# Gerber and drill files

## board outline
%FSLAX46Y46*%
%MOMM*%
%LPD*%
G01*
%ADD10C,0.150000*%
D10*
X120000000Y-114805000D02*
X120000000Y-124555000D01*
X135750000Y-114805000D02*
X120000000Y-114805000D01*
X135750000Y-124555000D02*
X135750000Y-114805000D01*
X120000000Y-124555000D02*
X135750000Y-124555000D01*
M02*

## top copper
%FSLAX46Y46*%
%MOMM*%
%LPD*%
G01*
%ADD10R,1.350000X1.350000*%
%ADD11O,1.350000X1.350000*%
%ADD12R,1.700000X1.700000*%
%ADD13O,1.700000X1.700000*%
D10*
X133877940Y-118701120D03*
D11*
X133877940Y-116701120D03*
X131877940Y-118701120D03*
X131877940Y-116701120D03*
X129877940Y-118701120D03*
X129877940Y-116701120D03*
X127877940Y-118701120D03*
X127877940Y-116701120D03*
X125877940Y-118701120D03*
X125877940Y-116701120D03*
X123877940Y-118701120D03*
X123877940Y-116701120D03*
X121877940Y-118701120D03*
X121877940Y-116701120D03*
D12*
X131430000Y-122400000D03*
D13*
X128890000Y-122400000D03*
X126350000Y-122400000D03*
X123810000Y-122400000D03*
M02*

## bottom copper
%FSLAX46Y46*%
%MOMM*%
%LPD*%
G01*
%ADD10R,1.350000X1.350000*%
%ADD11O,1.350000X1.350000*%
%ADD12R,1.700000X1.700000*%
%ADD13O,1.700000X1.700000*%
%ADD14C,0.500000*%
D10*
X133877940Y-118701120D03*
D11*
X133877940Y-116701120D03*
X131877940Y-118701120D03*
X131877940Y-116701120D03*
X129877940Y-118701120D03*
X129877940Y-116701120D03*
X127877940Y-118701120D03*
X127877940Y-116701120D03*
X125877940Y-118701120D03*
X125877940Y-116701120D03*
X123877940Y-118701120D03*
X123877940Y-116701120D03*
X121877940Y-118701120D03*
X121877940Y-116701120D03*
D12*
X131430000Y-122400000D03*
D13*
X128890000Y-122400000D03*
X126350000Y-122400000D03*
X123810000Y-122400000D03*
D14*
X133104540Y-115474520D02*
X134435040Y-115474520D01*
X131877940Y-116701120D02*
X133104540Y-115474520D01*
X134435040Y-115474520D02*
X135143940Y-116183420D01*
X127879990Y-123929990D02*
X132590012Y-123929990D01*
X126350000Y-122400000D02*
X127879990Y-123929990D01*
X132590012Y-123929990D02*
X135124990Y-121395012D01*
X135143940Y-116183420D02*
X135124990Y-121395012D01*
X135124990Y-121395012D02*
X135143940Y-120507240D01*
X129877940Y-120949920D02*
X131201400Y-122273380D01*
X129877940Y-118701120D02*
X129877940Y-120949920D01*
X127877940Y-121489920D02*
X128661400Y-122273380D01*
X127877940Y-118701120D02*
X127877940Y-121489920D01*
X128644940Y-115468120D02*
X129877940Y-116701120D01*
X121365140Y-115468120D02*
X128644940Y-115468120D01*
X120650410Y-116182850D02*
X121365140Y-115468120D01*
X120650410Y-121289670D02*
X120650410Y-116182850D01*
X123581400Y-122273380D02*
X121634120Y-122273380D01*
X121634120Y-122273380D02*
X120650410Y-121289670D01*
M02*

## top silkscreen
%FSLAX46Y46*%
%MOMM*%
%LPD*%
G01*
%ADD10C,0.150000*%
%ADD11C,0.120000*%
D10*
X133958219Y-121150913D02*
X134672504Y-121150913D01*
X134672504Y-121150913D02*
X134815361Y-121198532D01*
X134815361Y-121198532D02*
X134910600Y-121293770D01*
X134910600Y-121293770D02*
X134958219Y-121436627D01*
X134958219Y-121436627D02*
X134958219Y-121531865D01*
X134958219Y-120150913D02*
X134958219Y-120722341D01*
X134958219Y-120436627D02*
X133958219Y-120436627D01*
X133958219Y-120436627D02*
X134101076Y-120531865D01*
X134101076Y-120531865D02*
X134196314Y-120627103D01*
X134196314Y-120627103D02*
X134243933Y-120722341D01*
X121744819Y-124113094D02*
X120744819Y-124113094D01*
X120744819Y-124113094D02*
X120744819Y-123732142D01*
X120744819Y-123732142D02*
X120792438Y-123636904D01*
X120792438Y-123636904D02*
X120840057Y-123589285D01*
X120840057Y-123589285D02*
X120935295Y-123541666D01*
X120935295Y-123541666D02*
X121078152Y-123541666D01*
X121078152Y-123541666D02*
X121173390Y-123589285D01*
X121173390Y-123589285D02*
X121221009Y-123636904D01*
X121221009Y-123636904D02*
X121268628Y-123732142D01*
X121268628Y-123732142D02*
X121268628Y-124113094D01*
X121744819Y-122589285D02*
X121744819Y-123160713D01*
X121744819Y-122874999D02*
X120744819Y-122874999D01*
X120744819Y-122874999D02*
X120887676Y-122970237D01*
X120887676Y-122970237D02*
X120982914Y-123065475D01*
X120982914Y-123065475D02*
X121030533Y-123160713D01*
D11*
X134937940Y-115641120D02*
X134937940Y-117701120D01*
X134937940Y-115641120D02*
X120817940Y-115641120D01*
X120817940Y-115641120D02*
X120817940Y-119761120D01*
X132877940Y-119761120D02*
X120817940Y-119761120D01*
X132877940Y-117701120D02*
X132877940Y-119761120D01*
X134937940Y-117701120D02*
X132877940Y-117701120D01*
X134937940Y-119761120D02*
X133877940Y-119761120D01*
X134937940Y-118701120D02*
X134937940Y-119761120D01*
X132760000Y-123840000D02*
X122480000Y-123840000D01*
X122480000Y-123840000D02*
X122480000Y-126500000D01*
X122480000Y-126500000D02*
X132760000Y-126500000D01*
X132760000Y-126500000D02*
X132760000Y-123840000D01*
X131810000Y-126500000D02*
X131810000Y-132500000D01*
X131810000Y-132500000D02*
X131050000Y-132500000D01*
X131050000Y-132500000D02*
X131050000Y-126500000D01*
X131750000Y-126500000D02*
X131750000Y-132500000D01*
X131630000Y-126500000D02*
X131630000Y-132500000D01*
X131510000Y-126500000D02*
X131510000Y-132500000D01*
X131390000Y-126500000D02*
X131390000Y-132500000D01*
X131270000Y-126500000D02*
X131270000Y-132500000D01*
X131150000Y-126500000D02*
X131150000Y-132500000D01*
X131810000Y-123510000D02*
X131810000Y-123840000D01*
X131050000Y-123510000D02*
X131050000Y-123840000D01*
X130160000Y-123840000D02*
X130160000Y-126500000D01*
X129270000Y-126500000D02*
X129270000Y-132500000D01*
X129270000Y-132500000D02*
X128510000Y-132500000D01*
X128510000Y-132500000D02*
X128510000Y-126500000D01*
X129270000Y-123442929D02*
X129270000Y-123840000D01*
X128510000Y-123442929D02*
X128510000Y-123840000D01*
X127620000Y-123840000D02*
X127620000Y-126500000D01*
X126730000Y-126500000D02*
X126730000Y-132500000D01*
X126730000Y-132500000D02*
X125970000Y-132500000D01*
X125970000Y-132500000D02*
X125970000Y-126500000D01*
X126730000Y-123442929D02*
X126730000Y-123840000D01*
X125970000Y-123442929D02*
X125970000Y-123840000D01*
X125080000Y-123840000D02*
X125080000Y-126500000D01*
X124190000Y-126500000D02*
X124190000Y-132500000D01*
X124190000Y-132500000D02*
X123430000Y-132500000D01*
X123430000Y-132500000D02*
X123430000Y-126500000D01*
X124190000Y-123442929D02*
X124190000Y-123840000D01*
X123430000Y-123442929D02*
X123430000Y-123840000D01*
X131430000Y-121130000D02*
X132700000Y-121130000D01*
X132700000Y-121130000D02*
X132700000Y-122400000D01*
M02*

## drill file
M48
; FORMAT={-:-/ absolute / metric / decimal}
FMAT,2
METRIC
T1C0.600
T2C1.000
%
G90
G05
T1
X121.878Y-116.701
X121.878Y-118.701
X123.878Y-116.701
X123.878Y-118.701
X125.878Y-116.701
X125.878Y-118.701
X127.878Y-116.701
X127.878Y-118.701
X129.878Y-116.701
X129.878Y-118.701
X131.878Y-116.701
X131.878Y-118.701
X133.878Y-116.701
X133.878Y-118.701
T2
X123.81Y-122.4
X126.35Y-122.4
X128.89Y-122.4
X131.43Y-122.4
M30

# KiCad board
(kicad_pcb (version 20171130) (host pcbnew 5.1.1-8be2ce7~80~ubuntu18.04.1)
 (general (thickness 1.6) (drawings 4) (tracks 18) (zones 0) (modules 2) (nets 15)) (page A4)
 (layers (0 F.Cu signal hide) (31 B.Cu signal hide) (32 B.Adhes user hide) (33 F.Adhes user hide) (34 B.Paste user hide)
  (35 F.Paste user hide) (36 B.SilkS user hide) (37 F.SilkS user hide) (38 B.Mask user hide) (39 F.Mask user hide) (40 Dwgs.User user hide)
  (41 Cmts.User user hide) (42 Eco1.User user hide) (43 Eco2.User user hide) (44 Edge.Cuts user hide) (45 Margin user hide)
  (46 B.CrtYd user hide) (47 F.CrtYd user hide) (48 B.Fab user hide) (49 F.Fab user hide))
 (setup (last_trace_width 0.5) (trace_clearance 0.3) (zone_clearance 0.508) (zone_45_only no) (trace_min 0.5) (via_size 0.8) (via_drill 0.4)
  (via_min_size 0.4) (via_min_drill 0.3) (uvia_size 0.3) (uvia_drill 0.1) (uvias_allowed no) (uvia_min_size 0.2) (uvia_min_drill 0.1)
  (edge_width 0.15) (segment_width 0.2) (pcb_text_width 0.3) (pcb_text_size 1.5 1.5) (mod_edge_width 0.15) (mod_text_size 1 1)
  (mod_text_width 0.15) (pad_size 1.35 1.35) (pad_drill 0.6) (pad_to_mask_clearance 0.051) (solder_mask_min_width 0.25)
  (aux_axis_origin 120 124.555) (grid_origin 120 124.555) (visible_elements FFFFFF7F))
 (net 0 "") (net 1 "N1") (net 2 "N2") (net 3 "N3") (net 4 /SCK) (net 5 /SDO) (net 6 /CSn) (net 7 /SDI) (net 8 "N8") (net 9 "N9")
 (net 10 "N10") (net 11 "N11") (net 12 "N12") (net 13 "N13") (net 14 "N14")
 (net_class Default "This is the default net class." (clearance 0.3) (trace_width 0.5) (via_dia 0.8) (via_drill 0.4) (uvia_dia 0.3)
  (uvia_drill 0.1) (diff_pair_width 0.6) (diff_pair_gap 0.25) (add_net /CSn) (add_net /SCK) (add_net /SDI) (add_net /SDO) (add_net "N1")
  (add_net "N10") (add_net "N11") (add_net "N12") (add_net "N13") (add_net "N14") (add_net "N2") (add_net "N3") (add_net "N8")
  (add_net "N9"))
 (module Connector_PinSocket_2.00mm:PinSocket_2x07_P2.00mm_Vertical (layer F.Cu) (at 133.87794 118.70112 270)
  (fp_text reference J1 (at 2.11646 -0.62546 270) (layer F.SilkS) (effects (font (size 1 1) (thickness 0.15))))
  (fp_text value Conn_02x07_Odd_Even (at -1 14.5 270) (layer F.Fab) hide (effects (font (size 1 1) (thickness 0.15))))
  (fp_line (start -3.06 -1.06) (end -1 -1.06) (layer F.SilkS) (width 0.12))
  (fp_line (start -3.06 -1.06) (end -3.06 13.06) (layer F.SilkS) (width 0.12))
  (fp_line (start -3.06 13.06) (end 1.06 13.06) (layer F.SilkS) (width 0.12))
  (fp_line (start 1.06 1) (end 1.06 13.06) (layer F.SilkS) (width 0.12))
  (fp_line (start -1 1) (end 1.06 1) (layer F.SilkS) (width 0.12))
  (fp_line (start -1 -1.06) (end -1 1) (layer F.SilkS) (width 0.12))
  (fp_line (start 1.06 -1.06) (end 1.06 0) (layer F.SilkS) (width 0.12))
  (fp_line (start 0 -1.06) (end 1.06 -1.06) (layer F.SilkS) (width 0.12))
  (pad 1 thru_hole rect (at 0 0 270) (size 1.35 1.35) (drill 0.6) (layers *.Cu *.Mask) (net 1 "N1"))
  (pad 2 thru_hole oval (at -2 0 270) (size 1.35 1.35) (drill 0.6) (layers *.Cu *.Mask) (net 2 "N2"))
  (pad 3 thru_hole oval (at 0 2 270) (size 1.35 1.35) (drill 0.6) (layers *.Cu *.Mask) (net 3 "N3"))
  (pad 4 thru_hole oval (at -2 2 270) (size 1.35 1.35) (drill 0.6) (layers *.Cu *.Mask) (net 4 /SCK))
  (pad 5 thru_hole oval (at 0 4 270) (size 1.35 1.35) (drill 0.6) (layers *.Cu *.Mask) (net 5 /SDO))
  (pad 6 thru_hole oval (at -2 4 270) (size 1.35 1.35) (drill 0.6) (layers *.Cu *.Mask) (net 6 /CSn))
  (pad 7 thru_hole oval (at 0 6 270) (size 1.35 1.35) (drill 0.6) (layers *.Cu *.Mask) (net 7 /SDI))
  (pad 8 thru_hole oval (at -2 6 270) (size 1.35 1.35) (drill 0.6) (layers *.Cu *.Mask) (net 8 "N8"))
  (pad 9 thru_hole oval (at 0 8 270) (size 1.35 1.35) (drill 0.6) (layers *.Cu *.Mask) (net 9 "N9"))
  (pad 10 thru_hole oval (at -2 8 270) (size 1.35 1.35) (drill 0.6) (layers *.Cu *.Mask) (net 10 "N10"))
  (pad 11 thru_hole oval (at 0 10 270) (size 1.35 1.35) (drill 0.6) (layers *.Cu *.Mask) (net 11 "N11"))
  (pad 12 thru_hole oval (at -2 10 270) (size 1.35 1.35) (drill 0.6) (layers *.Cu *.Mask) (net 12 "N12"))
  (pad 13 thru_hole oval (at 0 12 270) (size 1.35 1.35) (drill 0.6) (layers *.Cu *.Mask) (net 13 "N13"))
  (pad 14 thru_hole oval (at -2 12 270) (size 1.35 1.35) (drill 0.6) (layers *.Cu *.Mask) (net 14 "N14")))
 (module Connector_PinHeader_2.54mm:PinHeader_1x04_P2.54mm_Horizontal (layer F.Cu) (at 131.43 122.4 270)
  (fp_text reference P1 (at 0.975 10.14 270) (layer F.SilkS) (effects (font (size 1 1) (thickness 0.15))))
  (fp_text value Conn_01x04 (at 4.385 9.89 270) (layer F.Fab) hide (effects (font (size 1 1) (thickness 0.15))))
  (fp_line (start 1.44 -1.33) (end 1.44 8.95) (layer F.SilkS) (width 0.12))
  (fp_line (start 1.44 8.95) (end 4.1 8.95) (layer F.SilkS) (width 0.12))
  (fp_line (start 4.1 8.95) (end 4.1 -1.33) (layer F.SilkS) (width 0.12))
  (fp_line (start 4.1 -1.33) (end 1.44 -1.33) (layer F.SilkS) (width 0.12))
  (fp_line (start 4.1 -0.38) (end 10.1 -0.38) (layer F.SilkS) (width 0.12))
  (fp_line (start 10.1 -0.38) (end 10.1 0.38) (layer F.SilkS) (width 0.12))
  (fp_line (start 10.1 0.38) (end 4.1 0.38) (layer F.SilkS) (width 0.12))
  (fp_line (start 4.1 -0.32) (end 10.1 -0.32) (layer F.SilkS) (width 0.12))
  (fp_line (start 4.1 -0.2) (end 10.1 -0.2) (layer F.SilkS) (width 0.12))
  (fp_line (start 4.1 -0.08) (end 10.1 -0.08) (layer F.SilkS) (width 0.12))
  (fp_line (start 4.1 0.04) (end 10.1 0.04) (layer F.SilkS) (width 0.12))
  (fp_line (start 4.1 0.16) (end 10.1 0.16) (layer F.SilkS) (width 0.12))
  (fp_line (start 4.1 0.28) (end 10.1 0.28) (layer F.SilkS) (width 0.12))
  (fp_line (start 1.11 -0.38) (end 1.44 -0.38) (layer F.SilkS) (width 0.12))
  (fp_line (start 1.11 0.38) (end 1.44 0.38) (layer F.SilkS) (width 0.12))
  (fp_line (start 1.44 1.27) (end 4.1 1.27) (layer F.SilkS) (width 0.12))
  (fp_line (start 4.1 2.16) (end 10.1 2.16) (layer F.SilkS) (width 0.12))
  (fp_line (start 10.1 2.16) (end 10.1 2.92) (layer F.SilkS) (width 0.12))
  (fp_line (start 10.1 2.92) (end 4.1 2.92) (layer F.SilkS) (width 0.12))
  (fp_line (start 1.042929 2.16) (end 1.44 2.16) (layer F.SilkS) (width 0.12))
  (fp_line (start 1.042929 2.92) (end 1.44 2.92) (layer F.SilkS) (width 0.12))
  (fp_line (start 1.44 3.81) (end 4.1 3.81) (layer F.SilkS) (width 0.12))
  (fp_line (start 4.1 4.7) (end 10.1 4.7) (layer F.SilkS) (width 0.12))
  (fp_line (start 10.1 4.7) (end 10.1 5.46) (layer F.SilkS) (width 0.12))
  (fp_line (start 10.1 5.46) (end 4.1 5.46) (layer F.SilkS) (width 0.12))
  (fp_line (start 1.042929 4.7) (end 1.44 4.7) (layer F.SilkS) (width 0.12))
  (fp_line (start 1.042929 5.46) (end 1.44 5.46) (layer F.SilkS) (width 0.12))
  (fp_line (start 1.44 6.35) (end 4.1 6.35) (layer F.SilkS) (width 0.12))
  (fp_line (start 4.1 7.24) (end 10.1 7.24) (layer F.SilkS) (width 0.12))
  (fp_line (start 10.1 7.24) (end 10.1 8) (layer F.SilkS) (width 0.12))
  (fp_line (start 10.1 8) (end 4.1 8) (layer F.SilkS) (width 0.12))
  (fp_line (start 1.042929 7.24) (end 1.44 7.24) (layer F.SilkS) (width 0.12))
  (fp_line (start 1.042929 8) (end 1.44 8) (layer F.SilkS) (width 0.12))
  (fp_line (start -1.27 0) (end -1.27 -1.27) (layer F.SilkS) (width 0.12))
  (fp_line (start -1.27 -1.27) (end 0 -1.27) (layer F.SilkS) (width 0.12))
  (pad 1 thru_hole rect (at 0 0 270) (size 1.7 1.7) (drill 1) (layers *.Cu *.Mask) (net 5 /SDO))
  (pad 2 thru_hole oval (at 0 2.54 270) (size 1.7 1.7) (drill 1) (layers *.Cu *.Mask) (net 7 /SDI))
  (pad 3 thru_hole oval (at 0 5.08 270) (size 1.7 1.7) (drill 1) (layers *.Cu *.Mask) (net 4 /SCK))
  (pad 4 thru_hole oval (at 0 7.62 270) (size 1.7 1.7) (drill 1) (layers *.Cu *.Mask) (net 6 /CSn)))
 (gr_line (start 120 114.805) (end 120 124.555) (layer Edge.Cuts) (width 0.15))
 (gr_line (start 135.75 114.805) (end 120 114.805) (layer Edge.Cuts) (width 0.15))
 (gr_line (start 135.75 124.555) (end 135.75 114.805) (layer Edge.Cuts) (width 0.15))
 (gr_line (start 120 124.555) (end 135.75 124.555) (layer Edge.Cuts) (width 0.15))
 (segment (start 133.10454 115.47452) (end 134.43504 115.47452) (width 0.5) (layer B.Cu) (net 4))
 (segment (start 131.87794 116.70112) (end 133.10454 115.47452) (width 0.5) (layer B.Cu) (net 4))
 (segment (start 134.43504 115.47452) (end 135.14394 116.18342) (width 0.5) (layer B.Cu) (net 4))
 (segment (start 127.87999 123.92999) (end 132.590012 123.92999) (width 0.5) (layer B.Cu) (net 4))
 (segment (start 126.35 122.4) (end 127.87999 123.92999) (width 0.5) (layer B.Cu) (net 4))
 (segment (start 132.590012 123.92999) (end 135.12499 121.395012) (width 0.5) (layer B.Cu) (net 4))
 (segment (start 135.14394 116.18342) (end 135.12499 121.395012) (width 0.5) (layer B.Cu) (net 4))
 (segment (start 135.12499 121.395012) (end 135.14394 120.50724) (width 0.5) (layer B.Cu) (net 4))
 (segment (start 129.87794 120.94992) (end 131.2014 122.27338) (width 0.5) (layer B.Cu) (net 5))
 (segment (start 129.87794 118.70112) (end 129.87794 120.94992) (width 0.5) (layer B.Cu) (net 5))
 (segment (start 127.87794 121.48992) (end 128.6614 122.27338) (width 0.5) (layer B.Cu) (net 7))
 (segment (start 127.87794 118.70112) (end 127.87794 121.48992) (width 0.5) (layer B.Cu) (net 7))
 (segment (start 128.64494 115.46812) (end 129.87794 116.70112) (width 0.5) (layer B.Cu) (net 6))
 (segment (start 121.36514 115.46812) (end 128.64494 115.46812) (width 0.5) (layer B.Cu) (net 6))
 (segment (start 120.65041 116.18285) (end 121.36514 115.46812) (width 0.5) (layer B.Cu) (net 6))
 (segment (start 120.65041 121.28967) (end 120.65041 116.18285) (width 0.5) (layer B.Cu) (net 6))
 (segment (start 123.5814 122.27338) (end 121.63412 122.27338) (width 0.5) (layer B.Cu) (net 6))
 (segment (start 121.63412 122.27338) (end 120.65041 121.28967) (width 0.5) (layer B.Cu) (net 6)))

